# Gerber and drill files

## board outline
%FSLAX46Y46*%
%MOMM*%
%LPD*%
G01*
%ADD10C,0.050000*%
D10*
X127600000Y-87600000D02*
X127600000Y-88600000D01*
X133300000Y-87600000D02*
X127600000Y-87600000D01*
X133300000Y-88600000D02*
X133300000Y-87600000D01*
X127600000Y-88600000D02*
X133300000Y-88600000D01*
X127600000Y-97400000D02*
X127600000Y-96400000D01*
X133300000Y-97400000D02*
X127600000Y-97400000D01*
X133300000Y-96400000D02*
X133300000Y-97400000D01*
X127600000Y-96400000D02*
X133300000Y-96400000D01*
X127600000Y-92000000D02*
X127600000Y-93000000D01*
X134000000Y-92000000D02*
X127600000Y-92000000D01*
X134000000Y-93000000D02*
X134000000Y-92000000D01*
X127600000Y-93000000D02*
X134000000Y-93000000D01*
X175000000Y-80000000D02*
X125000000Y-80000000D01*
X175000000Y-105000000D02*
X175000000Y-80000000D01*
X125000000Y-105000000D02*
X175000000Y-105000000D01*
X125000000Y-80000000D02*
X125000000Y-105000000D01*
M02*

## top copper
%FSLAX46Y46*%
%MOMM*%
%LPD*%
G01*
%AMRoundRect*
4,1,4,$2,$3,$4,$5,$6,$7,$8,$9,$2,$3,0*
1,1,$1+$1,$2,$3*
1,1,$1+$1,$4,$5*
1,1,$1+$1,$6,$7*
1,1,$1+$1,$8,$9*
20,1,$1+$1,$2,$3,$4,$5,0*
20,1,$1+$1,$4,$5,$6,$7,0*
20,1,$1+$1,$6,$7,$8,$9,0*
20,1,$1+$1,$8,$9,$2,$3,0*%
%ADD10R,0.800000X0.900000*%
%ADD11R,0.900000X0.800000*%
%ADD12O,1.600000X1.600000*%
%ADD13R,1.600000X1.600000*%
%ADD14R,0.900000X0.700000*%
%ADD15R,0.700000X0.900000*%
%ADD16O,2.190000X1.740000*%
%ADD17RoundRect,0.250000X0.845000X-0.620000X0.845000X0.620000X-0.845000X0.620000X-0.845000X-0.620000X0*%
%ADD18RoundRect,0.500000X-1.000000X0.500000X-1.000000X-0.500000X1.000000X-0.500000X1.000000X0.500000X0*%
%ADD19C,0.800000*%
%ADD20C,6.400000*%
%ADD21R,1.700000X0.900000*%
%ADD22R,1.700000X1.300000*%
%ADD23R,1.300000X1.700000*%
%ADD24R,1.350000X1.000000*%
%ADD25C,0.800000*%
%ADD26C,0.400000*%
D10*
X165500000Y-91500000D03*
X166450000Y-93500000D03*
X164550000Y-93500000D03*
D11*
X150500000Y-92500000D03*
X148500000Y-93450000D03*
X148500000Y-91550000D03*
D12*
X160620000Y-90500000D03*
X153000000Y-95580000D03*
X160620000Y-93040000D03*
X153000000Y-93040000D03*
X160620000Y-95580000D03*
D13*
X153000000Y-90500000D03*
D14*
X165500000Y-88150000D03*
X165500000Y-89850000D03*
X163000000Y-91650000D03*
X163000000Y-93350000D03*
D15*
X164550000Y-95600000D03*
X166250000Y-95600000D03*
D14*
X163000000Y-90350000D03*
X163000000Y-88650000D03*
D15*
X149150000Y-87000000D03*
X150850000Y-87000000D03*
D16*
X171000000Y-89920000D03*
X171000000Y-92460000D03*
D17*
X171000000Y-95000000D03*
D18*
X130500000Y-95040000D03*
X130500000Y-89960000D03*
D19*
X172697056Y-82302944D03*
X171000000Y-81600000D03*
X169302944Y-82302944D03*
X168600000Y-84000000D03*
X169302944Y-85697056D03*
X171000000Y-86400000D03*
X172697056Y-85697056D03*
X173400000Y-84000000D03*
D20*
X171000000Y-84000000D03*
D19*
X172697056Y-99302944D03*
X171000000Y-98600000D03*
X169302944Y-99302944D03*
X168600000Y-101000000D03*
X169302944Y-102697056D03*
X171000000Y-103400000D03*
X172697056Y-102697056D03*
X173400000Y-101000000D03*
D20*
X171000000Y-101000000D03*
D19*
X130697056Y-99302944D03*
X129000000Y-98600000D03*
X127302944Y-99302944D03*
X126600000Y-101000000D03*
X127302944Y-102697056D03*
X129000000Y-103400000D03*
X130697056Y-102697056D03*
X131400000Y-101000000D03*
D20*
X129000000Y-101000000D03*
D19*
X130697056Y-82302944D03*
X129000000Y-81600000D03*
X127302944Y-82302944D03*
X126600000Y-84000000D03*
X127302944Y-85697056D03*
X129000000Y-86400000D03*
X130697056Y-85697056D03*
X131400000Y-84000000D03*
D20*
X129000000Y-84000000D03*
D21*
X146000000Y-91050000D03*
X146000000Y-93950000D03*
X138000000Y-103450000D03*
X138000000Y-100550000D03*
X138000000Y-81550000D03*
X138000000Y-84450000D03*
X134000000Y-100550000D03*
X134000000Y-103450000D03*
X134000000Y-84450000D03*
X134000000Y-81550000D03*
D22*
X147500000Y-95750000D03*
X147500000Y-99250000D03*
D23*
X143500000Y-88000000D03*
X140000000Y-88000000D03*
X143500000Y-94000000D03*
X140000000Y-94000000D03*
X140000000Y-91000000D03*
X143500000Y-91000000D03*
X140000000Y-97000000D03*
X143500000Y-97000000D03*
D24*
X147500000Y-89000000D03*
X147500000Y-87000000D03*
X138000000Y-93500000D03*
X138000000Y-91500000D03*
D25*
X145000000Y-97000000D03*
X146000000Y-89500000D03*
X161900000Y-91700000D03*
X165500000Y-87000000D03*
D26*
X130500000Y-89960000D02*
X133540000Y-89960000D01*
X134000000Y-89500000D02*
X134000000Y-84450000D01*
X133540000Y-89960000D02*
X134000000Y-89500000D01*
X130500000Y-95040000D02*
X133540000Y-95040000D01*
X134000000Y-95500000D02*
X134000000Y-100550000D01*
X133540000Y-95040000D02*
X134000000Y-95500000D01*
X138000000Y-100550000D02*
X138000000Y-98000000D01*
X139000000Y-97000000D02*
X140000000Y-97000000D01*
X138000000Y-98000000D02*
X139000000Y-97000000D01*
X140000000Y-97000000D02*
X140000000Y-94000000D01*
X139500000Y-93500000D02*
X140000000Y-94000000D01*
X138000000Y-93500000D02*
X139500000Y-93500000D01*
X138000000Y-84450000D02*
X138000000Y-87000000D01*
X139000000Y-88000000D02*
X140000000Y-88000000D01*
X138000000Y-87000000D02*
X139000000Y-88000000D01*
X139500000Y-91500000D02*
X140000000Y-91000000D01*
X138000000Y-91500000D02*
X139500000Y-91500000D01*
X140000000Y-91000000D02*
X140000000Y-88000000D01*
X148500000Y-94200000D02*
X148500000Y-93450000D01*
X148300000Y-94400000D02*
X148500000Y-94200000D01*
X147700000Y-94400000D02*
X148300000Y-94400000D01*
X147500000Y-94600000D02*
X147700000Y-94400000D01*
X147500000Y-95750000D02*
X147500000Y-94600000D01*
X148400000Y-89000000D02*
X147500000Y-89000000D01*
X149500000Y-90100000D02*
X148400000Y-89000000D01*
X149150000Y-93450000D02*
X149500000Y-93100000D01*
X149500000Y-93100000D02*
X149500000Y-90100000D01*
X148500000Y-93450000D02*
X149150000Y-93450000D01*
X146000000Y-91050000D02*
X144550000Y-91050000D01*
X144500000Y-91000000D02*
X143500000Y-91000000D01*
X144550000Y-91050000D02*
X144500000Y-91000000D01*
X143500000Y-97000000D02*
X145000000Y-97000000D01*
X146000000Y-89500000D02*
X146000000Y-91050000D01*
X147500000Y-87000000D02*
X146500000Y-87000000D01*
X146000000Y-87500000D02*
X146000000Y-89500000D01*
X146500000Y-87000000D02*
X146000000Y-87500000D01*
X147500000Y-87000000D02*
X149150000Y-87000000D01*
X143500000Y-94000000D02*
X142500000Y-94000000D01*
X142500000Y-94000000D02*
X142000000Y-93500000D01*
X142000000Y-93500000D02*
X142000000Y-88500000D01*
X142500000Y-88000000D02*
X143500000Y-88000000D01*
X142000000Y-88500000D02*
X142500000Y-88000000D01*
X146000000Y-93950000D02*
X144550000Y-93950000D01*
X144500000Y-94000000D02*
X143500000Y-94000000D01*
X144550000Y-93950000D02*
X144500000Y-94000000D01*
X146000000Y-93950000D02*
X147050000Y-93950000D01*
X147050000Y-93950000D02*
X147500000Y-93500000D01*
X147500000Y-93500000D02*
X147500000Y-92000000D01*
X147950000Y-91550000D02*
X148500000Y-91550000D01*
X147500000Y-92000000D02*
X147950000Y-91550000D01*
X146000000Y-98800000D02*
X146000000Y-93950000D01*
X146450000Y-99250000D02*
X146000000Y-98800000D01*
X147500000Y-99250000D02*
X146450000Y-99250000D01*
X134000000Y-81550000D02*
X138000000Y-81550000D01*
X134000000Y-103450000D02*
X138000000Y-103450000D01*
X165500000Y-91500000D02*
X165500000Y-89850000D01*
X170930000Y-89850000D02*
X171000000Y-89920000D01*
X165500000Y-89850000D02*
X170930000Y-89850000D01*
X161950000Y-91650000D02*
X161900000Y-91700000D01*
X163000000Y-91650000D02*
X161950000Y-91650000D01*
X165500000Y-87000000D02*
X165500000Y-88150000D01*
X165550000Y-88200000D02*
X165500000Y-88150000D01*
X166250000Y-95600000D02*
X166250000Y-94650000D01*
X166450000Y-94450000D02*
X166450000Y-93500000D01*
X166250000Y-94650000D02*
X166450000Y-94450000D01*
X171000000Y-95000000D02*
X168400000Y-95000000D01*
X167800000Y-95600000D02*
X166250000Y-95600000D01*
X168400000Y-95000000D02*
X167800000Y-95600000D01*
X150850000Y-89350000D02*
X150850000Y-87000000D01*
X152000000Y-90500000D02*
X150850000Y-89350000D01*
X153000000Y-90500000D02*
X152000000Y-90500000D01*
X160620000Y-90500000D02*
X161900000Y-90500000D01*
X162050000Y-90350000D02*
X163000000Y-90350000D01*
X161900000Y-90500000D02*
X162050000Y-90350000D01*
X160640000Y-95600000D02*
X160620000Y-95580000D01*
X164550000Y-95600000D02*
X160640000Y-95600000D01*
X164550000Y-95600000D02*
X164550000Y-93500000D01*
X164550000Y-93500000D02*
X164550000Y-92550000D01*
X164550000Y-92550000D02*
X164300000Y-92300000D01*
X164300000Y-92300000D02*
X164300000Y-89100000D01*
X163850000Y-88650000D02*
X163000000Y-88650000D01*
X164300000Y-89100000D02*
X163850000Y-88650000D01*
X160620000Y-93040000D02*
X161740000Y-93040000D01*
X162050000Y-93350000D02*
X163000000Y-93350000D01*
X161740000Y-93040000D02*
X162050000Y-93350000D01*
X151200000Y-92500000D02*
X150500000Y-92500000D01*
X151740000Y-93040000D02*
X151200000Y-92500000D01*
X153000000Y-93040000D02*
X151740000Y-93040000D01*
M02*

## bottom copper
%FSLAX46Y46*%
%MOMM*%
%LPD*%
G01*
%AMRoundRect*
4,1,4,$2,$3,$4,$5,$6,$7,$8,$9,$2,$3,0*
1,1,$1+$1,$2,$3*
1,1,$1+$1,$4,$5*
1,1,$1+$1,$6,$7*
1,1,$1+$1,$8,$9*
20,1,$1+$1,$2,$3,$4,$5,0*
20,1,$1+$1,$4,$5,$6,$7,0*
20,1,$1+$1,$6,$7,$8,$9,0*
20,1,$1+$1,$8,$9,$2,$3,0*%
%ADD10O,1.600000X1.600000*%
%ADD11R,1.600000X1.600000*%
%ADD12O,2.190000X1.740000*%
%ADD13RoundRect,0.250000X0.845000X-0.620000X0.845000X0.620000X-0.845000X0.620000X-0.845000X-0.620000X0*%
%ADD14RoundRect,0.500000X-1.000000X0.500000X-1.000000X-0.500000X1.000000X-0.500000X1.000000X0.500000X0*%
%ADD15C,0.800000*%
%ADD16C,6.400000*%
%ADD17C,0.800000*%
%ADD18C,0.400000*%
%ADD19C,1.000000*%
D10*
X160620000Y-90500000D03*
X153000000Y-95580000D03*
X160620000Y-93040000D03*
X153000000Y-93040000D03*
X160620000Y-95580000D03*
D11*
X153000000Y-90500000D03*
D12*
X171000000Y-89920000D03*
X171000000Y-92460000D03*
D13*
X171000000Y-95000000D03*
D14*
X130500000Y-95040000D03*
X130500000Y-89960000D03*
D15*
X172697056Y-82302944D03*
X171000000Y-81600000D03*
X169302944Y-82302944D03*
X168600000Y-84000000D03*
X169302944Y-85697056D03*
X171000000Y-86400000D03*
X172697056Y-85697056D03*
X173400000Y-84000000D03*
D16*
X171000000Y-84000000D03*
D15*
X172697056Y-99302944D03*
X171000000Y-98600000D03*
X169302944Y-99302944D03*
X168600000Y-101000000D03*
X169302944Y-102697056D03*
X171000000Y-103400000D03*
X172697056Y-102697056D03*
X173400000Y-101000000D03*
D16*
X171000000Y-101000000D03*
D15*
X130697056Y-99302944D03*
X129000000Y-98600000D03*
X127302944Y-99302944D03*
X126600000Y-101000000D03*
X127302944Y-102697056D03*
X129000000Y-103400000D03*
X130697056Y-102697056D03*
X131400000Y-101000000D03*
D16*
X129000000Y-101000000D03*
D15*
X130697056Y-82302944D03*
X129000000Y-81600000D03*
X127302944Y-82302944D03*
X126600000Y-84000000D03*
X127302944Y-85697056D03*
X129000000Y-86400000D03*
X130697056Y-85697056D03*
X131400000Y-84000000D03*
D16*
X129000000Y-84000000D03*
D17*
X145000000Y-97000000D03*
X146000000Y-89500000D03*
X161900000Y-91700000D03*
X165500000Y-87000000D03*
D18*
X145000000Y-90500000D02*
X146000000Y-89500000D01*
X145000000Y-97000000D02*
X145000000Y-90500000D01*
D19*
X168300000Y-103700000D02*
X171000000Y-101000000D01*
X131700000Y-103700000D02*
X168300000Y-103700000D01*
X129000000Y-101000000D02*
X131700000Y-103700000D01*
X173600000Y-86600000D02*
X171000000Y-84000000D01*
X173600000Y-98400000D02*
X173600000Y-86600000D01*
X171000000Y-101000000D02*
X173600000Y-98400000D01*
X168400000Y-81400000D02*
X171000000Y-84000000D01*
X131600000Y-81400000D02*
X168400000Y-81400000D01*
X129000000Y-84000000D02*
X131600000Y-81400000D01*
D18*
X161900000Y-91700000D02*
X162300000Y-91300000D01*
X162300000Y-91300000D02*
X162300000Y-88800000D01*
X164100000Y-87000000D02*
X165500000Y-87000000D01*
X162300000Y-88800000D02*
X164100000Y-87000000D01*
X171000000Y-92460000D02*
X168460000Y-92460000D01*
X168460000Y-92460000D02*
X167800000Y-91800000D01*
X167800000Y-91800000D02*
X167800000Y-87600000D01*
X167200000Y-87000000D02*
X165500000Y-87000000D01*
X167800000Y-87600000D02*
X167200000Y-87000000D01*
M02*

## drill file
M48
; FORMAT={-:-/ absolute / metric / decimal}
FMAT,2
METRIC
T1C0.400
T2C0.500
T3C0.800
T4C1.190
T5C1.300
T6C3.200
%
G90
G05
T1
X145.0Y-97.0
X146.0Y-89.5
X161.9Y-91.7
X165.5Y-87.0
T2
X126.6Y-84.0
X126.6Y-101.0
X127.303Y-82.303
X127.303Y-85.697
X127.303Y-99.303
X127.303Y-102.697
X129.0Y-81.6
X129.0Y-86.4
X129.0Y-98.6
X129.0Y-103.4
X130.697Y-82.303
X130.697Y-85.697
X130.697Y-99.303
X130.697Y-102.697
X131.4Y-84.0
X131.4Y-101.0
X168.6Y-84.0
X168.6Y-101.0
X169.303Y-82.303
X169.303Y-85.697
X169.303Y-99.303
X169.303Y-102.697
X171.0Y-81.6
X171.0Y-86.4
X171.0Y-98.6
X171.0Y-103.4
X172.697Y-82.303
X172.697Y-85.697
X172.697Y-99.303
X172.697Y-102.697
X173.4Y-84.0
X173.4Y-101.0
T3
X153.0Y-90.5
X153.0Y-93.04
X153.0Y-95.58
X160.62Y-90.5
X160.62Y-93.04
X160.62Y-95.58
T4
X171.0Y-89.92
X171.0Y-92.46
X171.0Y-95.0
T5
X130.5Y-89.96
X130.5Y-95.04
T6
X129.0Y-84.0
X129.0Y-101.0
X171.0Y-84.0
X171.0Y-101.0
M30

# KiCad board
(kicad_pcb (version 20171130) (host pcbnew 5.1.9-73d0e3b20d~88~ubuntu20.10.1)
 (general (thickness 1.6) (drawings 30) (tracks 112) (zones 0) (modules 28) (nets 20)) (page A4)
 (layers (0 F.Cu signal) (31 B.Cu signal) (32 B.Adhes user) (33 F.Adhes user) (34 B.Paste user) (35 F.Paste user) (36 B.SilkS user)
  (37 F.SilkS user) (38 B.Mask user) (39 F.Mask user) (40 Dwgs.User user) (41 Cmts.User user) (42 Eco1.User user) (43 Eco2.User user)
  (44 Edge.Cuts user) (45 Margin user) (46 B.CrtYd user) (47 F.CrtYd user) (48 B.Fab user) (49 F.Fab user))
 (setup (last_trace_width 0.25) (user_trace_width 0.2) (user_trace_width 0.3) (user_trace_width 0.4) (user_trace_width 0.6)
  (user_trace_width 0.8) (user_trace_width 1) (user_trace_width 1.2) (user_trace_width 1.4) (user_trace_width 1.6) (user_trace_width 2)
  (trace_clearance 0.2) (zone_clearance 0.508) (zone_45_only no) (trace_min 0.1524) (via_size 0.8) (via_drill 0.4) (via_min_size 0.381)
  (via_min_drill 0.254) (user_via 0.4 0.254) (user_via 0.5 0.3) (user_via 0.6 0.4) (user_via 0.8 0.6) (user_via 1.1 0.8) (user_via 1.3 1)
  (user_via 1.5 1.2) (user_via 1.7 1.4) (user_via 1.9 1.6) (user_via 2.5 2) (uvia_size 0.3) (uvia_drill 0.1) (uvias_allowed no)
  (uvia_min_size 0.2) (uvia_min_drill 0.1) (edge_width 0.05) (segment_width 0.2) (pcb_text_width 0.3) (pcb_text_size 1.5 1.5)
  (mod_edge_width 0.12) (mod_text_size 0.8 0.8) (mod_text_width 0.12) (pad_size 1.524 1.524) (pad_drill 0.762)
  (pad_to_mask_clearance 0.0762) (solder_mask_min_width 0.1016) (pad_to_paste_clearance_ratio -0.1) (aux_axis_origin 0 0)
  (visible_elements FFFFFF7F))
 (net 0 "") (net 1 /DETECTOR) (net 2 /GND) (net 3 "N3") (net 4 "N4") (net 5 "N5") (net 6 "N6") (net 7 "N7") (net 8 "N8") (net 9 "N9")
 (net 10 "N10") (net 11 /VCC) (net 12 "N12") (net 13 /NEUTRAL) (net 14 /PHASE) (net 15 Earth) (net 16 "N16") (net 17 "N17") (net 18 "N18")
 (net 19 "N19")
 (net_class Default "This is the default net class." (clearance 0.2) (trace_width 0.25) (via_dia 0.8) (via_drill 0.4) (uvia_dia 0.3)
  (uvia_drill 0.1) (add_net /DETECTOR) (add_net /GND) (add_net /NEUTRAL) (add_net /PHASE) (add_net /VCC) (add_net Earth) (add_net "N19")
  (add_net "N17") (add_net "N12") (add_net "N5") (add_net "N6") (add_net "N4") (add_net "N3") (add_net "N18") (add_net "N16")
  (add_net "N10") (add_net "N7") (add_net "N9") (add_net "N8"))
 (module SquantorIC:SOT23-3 (layer F.Cu) (at 165.5 92.5)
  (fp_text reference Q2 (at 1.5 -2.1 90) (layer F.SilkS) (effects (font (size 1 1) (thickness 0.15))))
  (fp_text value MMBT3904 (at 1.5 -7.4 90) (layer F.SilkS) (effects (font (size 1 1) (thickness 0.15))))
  (pad 3 smd rect (at 0 -1) (size 0.8 0.9) (layers F.Cu F.Paste F.Mask) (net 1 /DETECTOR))
  (pad 2 smd rect (at 0.95 1) (size 0.8 0.9) (layers F.Cu F.Paste F.Mask) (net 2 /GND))
  (pad 1 smd rect (at -0.95 1) (size 0.8 0.9) (layers F.Cu F.Paste F.Mask) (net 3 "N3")))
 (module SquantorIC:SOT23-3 (layer F.Cu) (at 149.5 92.5 270)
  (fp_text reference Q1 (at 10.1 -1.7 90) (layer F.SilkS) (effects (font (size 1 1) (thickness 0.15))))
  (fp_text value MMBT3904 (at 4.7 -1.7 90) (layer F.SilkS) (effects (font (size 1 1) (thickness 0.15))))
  (pad 3 smd rect (at 0 -1 270) (size 0.8 0.9) (layers F.Cu F.Paste F.Mask) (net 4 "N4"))
  (pad 2 smd rect (at 0.95 1 270) (size 0.8 0.9) (layers F.Cu F.Paste F.Mask) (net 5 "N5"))
  (pad 1 smd rect (at -0.95 1 270) (size 0.8 0.9) (layers F.Cu F.Paste F.Mask) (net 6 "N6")))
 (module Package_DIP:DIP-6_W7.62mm (layer F.Cu) (at 153 90.5)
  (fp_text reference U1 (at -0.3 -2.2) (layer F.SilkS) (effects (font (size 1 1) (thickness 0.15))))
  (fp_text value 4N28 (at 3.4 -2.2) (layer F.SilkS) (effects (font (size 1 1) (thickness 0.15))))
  (pad 6 thru_hole oval (at 7.62 0) (size 1.6 1.6) (drill 0.8) (layers *.Cu *.Mask) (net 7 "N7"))
  (pad 3 thru_hole oval (at 0 5.08) (size 1.6 1.6) (drill 0.8) (layers *.Cu *.Mask) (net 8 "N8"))
  (pad 5 thru_hole oval (at 7.62 2.54) (size 1.6 1.6) (drill 0.8) (layers *.Cu *.Mask) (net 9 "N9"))
  (pad 2 thru_hole oval (at 0 2.54) (size 1.6 1.6) (drill 0.8) (layers *.Cu *.Mask) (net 4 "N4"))
  (pad 4 thru_hole oval (at 7.62 5.08) (size 1.6 1.6) (drill 0.8) (layers *.Cu *.Mask) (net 3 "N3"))
  (pad 1 thru_hole rect (at 0 0) (size 1.6 1.6) (drill 0.8) (layers *.Cu *.Mask) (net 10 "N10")))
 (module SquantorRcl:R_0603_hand (layer F.Cu) (at 165.5 89 90)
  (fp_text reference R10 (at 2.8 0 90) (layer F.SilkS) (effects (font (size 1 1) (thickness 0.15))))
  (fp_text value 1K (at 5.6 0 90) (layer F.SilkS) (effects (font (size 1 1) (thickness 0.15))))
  (pad 2 smd rect (at 0.85 0 90) (size 0.7 0.9) (layers F.Cu F.Paste F.Mask) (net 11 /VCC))
  (pad 1 smd rect (at -0.85 0 90) (size 0.7 0.9) (layers F.Cu F.Paste F.Mask) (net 1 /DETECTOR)))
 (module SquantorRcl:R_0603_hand (layer F.Cu) (at 163 92.5 90)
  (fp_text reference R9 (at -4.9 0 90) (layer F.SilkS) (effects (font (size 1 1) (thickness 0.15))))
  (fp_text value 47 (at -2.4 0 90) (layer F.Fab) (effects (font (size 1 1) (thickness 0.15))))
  (pad 2 smd rect (at 0.85 0 90) (size 0.7 0.9) (layers F.Cu F.Paste F.Mask) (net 11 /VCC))
  (pad 1 smd rect (at -0.85 0 90) (size 0.7 0.9) (layers F.Cu F.Paste F.Mask) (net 9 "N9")))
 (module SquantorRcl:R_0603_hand (layer F.Cu) (at 165.4 95.6 180)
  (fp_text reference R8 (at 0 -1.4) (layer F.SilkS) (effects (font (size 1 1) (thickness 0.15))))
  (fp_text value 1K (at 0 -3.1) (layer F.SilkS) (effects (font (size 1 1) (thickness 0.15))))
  (pad 2 smd rect (at 0.85 0 180) (size 0.7 0.9) (layers F.Cu F.Paste F.Mask) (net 3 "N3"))
  (pad 1 smd rect (at -0.85 0 180) (size 0.7 0.9) (layers F.Cu F.Paste F.Mask) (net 2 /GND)))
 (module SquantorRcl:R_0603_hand (layer F.Cu) (at 163 89.5 270)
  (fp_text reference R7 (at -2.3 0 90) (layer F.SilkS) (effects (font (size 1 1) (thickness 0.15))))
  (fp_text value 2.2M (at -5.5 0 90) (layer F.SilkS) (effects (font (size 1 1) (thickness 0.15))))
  (pad 2 smd rect (at 0.85 0 270) (size 0.7 0.9) (layers F.Cu F.Paste F.Mask) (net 7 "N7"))
  (pad 1 smd rect (at -0.85 0 270) (size 0.7 0.9) (layers F.Cu F.Paste F.Mask) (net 3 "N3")))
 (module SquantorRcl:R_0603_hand (layer F.Cu) (at 150 87 180)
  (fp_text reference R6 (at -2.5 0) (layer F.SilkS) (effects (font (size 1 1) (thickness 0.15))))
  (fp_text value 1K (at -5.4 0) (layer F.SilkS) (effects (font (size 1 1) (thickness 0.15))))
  (pad 2 smd rect (at 0.85 0 180) (size 0.7 0.9) (layers F.Cu F.Paste F.Mask) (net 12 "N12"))
  (pad 1 smd rect (at -0.85 0 180) (size 0.7 0.9) (layers F.Cu F.Paste F.Mask) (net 10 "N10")))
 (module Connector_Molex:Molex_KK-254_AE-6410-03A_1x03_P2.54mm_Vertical (layer F.Cu) (at 171 95 90)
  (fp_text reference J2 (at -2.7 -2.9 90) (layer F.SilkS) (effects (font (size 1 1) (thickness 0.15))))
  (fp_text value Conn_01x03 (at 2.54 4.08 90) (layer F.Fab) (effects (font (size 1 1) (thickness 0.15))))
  (pad 3 thru_hole oval (at 5.08 0 90) (size 1.74 2.19) (drill 1.19) (layers *.Cu *.Mask) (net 1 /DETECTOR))
  (pad 2 thru_hole oval (at 2.54 0 90) (size 1.74 2.19) (drill 1.19) (layers *.Cu *.Mask) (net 11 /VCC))
  (pad 1 thru_hole roundrect (at 0 0 90) (size 1.74 2.19) (drill 1.19) (layers *.Cu *.Mask) (roundrect_rratio 0.143678) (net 2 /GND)))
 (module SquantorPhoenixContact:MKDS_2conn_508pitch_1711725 (layer F.Cu) (at 130.5 92.5 270)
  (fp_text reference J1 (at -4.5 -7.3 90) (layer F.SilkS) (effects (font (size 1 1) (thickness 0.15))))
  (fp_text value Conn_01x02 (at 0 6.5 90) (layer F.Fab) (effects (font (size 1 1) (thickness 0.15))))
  (pad 2 thru_hole roundrect (at 2.54 0 270) (size 2 3) (drill 1.3) (layers *.Cu *.Mask) (roundrect_rratio 0.25) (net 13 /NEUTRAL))
  (pad 1 thru_hole roundrect (at -2.54 0 270) (size 2 3) (drill 1.3) (layers *.Cu *.Mask) (roundrect_rratio 0.25) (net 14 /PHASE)))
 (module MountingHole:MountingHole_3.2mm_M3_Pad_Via (layer F.Cu) (at 171 84)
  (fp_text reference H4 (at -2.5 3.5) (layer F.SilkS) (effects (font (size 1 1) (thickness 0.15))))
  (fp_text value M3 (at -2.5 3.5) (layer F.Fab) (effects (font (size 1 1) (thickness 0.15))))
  (pad 1 thru_hole circle (at 1.697056 -1.697056) (size 0.8 0.8) (drill 0.5) (layers *.Cu *.Mask) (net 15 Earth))
  (pad 1 thru_hole circle (at 0 -2.4) (size 0.8 0.8) (drill 0.5) (layers *.Cu *.Mask) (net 15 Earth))
  (pad 1 thru_hole circle (at -1.697056 -1.697056) (size 0.8 0.8) (drill 0.5) (layers *.Cu *.Mask) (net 15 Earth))
  (pad 1 thru_hole circle (at -2.4 0) (size 0.8 0.8) (drill 0.5) (layers *.Cu *.Mask) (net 15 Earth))
  (pad 1 thru_hole circle (at -1.697056 1.697056) (size 0.8 0.8) (drill 0.5) (layers *.Cu *.Mask) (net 15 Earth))
  (pad 1 thru_hole circle (at 0 2.4) (size 0.8 0.8) (drill 0.5) (layers *.Cu *.Mask) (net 15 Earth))
  (pad 1 thru_hole circle (at 1.697056 1.697056) (size 0.8 0.8) (drill 0.5) (layers *.Cu *.Mask) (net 15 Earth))
  (pad 1 thru_hole circle (at 2.4 0) (size 0.8 0.8) (drill 0.5) (layers *.Cu *.Mask) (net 15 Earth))
  (pad 1 thru_hole circle (at 0 0) (size 6.4 6.4) (drill 3.2) (layers *.Cu *.Mask) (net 15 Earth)))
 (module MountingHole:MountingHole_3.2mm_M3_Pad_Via (layer F.Cu) (at 171 101)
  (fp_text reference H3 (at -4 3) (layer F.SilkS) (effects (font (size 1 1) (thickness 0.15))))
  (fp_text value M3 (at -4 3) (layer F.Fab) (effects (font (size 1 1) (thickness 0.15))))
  (pad 1 thru_hole circle (at 1.697056 -1.697056) (size 0.8 0.8) (drill 0.5) (layers *.Cu *.Mask) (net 15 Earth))
  (pad 1 thru_hole circle (at 0 -2.4) (size 0.8 0.8) (drill 0.5) (layers *.Cu *.Mask) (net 15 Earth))
  (pad 1 thru_hole circle (at -1.697056 -1.697056) (size 0.8 0.8) (drill 0.5) (layers *.Cu *.Mask) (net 15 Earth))
  (pad 1 thru_hole circle (at -2.4 0) (size 0.8 0.8) (drill 0.5) (layers *.Cu *.Mask) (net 15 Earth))
  (pad 1 thru_hole circle (at -1.697056 1.697056) (size 0.8 0.8) (drill 0.5) (layers *.Cu *.Mask) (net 15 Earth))
  (pad 1 thru_hole circle (at 0 2.4) (size 0.8 0.8) (drill 0.5) (layers *.Cu *.Mask) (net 15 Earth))
  (pad 1 thru_hole circle (at 1.697056 1.697056) (size 0.8 0.8) (drill 0.5) (layers *.Cu *.Mask) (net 15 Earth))
  (pad 1 thru_hole circle (at 2.4 0) (size 0.8 0.8) (drill 0.5) (layers *.Cu *.Mask) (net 15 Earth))
  (pad 1 thru_hole circle (at 0 0) (size 6.4 6.4) (drill 3.2) (layers *.Cu *.Mask) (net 15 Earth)))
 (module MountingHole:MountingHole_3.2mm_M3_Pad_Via (layer F.Cu) (at 129 101)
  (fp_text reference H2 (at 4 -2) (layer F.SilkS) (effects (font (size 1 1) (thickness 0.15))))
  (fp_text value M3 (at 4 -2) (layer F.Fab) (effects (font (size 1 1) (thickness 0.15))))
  (pad 1 thru_hole circle (at 1.697056 -1.697056) (size 0.8 0.8) (drill 0.5) (layers *.Cu *.Mask) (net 15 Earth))
  (pad 1 thru_hole circle (at 0 -2.4) (size 0.8 0.8) (drill 0.5) (layers *.Cu *.Mask) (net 15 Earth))
  (pad 1 thru_hole circle (at -1.697056 -1.697056) (size 0.8 0.8) (drill 0.5) (layers *.Cu *.Mask) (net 15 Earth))
  (pad 1 thru_hole circle (at -2.4 0) (size 0.8 0.8) (drill 0.5) (layers *.Cu *.Mask) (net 15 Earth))
  (pad 1 thru_hole circle (at -1.697056 1.697056) (size 0.8 0.8) (drill 0.5) (layers *.Cu *.Mask) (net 15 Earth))
  (pad 1 thru_hole circle (at 0 2.4) (size 0.8 0.8) (drill 0.5) (layers *.Cu *.Mask) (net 15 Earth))
  (pad 1 thru_hole circle (at 1.697056 1.697056) (size 0.8 0.8) (drill 0.5) (layers *.Cu *.Mask) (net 15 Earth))
  (pad 1 thru_hole circle (at 2.4 0) (size 0.8 0.8) (drill 0.5) (layers *.Cu *.Mask) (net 15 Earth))
  (pad 1 thru_hole circle (at 0 0) (size 6.4 6.4) (drill 3.2) (layers *.Cu *.Mask) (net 15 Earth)))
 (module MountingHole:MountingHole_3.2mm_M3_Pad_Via (layer F.Cu) (at 129 84)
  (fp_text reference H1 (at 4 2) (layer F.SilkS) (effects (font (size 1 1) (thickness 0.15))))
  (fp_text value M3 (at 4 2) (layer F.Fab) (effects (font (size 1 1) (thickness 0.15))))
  (pad 1 thru_hole circle (at 1.697056 -1.697056) (size 0.8 0.8) (drill 0.5) (layers *.Cu *.Mask) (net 15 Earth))
  (pad 1 thru_hole circle (at 0 -2.4) (size 0.8 0.8) (drill 0.5) (layers *.Cu *.Mask) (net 15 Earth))
  (pad 1 thru_hole circle (at -1.697056 -1.697056) (size 0.8 0.8) (drill 0.5) (layers *.Cu *.Mask) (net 15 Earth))
  (pad 1 thru_hole circle (at -2.4 0) (size 0.8 0.8) (drill 0.5) (layers *.Cu *.Mask) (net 15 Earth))
  (pad 1 thru_hole circle (at -1.697056 1.697056) (size 0.8 0.8) (drill 0.5) (layers *.Cu *.Mask) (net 15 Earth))
  (pad 1 thru_hole circle (at 0 2.4) (size 0.8 0.8) (drill 0.5) (layers *.Cu *.Mask) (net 15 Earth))
  (pad 1 thru_hole circle (at 1.697056 1.697056) (size 0.8 0.8) (drill 0.5) (layers *.Cu *.Mask) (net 15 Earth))
  (pad 1 thru_hole circle (at 2.4 0) (size 0.8 0.8) (drill 0.5) (layers *.Cu *.Mask) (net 15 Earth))
  (pad 1 thru_hole circle (at 0 0) (size 6.4 6.4) (drill 3.2) (layers *.Cu *.Mask) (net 15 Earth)))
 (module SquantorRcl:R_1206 (layer F.Cu) (at 146 92.5 90)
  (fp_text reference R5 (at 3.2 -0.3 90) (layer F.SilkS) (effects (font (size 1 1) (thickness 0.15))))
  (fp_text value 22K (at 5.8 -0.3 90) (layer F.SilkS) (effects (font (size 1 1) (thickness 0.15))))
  (pad 2 smd rect (at 1.45 0 90) (size 0.9 1.7) (layers F.Cu F.Paste F.Mask) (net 12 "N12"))
  (pad 1 smd rect (at -1.45 0 90) (size 0.9 1.7) (layers F.Cu F.Paste F.Mask) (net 6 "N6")))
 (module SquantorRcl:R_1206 (layer F.Cu) (at 138 102 270)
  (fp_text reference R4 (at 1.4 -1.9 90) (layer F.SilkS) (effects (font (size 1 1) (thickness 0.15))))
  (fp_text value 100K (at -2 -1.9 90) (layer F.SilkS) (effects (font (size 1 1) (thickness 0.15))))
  (pad 2 smd rect (at 1.45 0 270) (size 0.9 1.7) (layers F.Cu F.Paste F.Mask) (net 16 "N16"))
  (pad 1 smd rect (at -1.45 0 270) (size 0.9 1.7) (layers F.Cu F.Paste F.Mask) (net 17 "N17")))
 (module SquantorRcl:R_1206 (layer F.Cu) (at 138 83 90)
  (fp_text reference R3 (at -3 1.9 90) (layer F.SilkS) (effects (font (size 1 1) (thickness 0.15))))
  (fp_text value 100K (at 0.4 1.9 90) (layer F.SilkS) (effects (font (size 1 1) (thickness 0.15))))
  (pad 2 smd rect (at 1.45 0 90) (size 0.9 1.7) (layers F.Cu F.Paste F.Mask) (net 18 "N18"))
  (pad 1 smd rect (at -1.45 0 90) (size 0.9 1.7) (layers F.Cu F.Paste F.Mask) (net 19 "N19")))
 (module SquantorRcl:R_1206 (layer F.Cu) (at 134 102 90)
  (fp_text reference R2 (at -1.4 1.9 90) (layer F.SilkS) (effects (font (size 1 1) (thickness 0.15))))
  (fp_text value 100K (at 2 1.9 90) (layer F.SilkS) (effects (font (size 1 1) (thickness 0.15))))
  (pad 2 smd rect (at 1.45 0 90) (size 0.9 1.7) (layers F.Cu F.Paste F.Mask) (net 13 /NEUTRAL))
  (pad 1 smd rect (at -1.45 0 90) (size 0.9 1.7) (layers F.Cu F.Paste F.Mask) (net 16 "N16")))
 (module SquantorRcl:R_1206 (layer F.Cu) (at 134 83 270)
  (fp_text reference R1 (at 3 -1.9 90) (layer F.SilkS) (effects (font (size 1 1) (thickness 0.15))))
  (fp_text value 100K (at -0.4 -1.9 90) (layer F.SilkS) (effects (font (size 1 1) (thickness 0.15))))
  (pad 2 smd rect (at 1.45 0 270) (size 0.9 1.7) (layers F.Cu F.Paste F.Mask) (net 14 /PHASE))
  (pad 1 smd rect (at -1.45 0 270) (size 0.9 1.7) (layers F.Cu F.Paste F.Mask) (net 18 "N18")))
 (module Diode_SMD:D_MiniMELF (layer F.Cu) (at 147.5 97.5 90)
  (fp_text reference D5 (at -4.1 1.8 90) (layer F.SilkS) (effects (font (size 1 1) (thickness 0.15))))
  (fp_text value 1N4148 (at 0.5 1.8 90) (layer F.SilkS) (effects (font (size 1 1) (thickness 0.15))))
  (pad 2 smd rect (at 1.75 0 90) (size 1.3 1.7) (layers F.Cu F.Paste F.Mask) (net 5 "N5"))
  (pad 1 smd rect (at -1.75 0 90) (size 1.3 1.7) (layers F.Cu F.Paste F.Mask) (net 6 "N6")))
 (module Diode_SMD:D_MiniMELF (layer F.Cu) (at 141.75 88)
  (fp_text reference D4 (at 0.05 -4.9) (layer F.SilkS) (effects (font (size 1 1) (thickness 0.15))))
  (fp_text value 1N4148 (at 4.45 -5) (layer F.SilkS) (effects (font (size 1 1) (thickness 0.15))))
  (pad 2 smd rect (at 1.75 0) (size 1.3 1.7) (layers F.Cu F.Paste F.Mask) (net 6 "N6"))
  (pad 1 smd rect (at -1.75 0) (size 1.3 1.7) (layers F.Cu F.Paste F.Mask) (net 19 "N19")))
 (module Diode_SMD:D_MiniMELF (layer F.Cu) (at 141.75 94)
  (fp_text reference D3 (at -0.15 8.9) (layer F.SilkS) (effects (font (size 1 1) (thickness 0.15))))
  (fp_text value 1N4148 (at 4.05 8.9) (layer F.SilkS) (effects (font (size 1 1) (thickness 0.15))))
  (pad 2 smd rect (at 1.75 0) (size 1.3 1.7) (layers F.Cu F.Paste F.Mask) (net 6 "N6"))
  (pad 1 smd rect (at -1.75 0) (size 1.3 1.7) (layers F.Cu F.Paste F.Mask) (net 17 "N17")))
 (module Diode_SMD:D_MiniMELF (layer F.Cu) (at 141.75 91 180)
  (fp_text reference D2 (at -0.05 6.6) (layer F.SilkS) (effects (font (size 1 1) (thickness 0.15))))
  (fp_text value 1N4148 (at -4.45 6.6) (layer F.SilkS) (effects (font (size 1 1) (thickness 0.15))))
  (pad 2 smd rect (at 1.75 0 180) (size 1.3 1.7) (layers F.Cu F.Paste F.Mask) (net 19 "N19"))
  (pad 1 smd rect (at -1.75 0 180) (size 1.3 1.7) (layers F.Cu F.Paste F.Mask) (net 12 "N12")))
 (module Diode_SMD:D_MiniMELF (layer F.Cu) (at 141.75 97 180)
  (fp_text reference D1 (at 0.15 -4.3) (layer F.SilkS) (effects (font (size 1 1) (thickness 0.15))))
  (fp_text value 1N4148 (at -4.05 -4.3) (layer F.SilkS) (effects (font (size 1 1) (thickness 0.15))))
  (pad 2 smd rect (at 1.75 0 180) (size 1.3 1.7) (layers F.Cu F.Paste F.Mask) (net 17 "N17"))
  (pad 1 smd rect (at -1.75 0 180) (size 1.3 1.7) (layers F.Cu F.Paste F.Mask) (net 12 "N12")))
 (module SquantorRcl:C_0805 (layer F.Cu) (at 147.5 88 270)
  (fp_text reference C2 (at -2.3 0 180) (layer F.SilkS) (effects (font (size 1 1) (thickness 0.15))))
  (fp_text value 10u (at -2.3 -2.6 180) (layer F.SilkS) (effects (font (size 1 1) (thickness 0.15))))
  (pad 2 smd rect (at 1 0 270) (size 1 1.35) (layers F.Cu F.Paste F.Mask) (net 5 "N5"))
  (pad 1 smd rect (at -1 0 270) (size 1 1.35) (layers F.Cu F.Paste F.Mask) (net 12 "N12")))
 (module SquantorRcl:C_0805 (layer F.Cu) (at 138 92.5 270)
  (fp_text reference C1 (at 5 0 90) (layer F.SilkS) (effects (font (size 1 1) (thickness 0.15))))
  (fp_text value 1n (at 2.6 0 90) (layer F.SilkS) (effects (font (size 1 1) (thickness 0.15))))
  (pad 2 smd rect (at 1 0 270) (size 1 1.35) (layers F.Cu F.Paste F.Mask) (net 17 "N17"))
  (pad 1 smd rect (at -1 0 270) (size 1 1.35) (layers F.Cu F.Paste F.Mask) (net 19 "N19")))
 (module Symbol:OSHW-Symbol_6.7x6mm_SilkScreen (layer B.Cu) (at 156.9 98.7 180)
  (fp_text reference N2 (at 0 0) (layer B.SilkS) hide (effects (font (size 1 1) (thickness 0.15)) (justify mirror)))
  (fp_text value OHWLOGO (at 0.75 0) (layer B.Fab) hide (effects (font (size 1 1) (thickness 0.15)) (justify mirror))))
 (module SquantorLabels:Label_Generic (layer B.Cu) (at 157.5 102.6 180)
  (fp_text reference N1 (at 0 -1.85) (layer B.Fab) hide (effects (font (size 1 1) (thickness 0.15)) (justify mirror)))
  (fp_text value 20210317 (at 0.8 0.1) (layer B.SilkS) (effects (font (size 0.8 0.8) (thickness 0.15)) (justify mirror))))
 (gr_line (start 127.6 87.6) (end 127.6 88.6) (layer Edge.Cuts) (width 0.05))
 (gr_line (start 133.3 87.6) (end 127.6 87.6) (layer Edge.Cuts) (width 0.05))
 (gr_line (start 133.3 88.6) (end 133.3 87.6) (layer Edge.Cuts) (width 0.05))
 (gr_line (start 127.6 88.6) (end 133.3 88.6) (layer Edge.Cuts) (width 0.05))
 (gr_line (start 127.6 97.4) (end 127.6 96.4) (layer Edge.Cuts) (width 0.05))
 (gr_line (start 133.3 97.4) (end 127.6 97.4) (layer Edge.Cuts) (width 0.05))
 (gr_line (start 133.3 96.4) (end 133.3 97.4) (layer Edge.Cuts) (width 0.05))
 (gr_line (start 127.6 96.4) (end 133.3 96.4) (layer Edge.Cuts) (width 0.05))
 (gr_line (start 127.6 92) (end 127.6 93) (layer Edge.Cuts) (width 0.05))
 (gr_line (start 134 92) (end 127.6 92) (layer Edge.Cuts) (width 0.05))
 (gr_line (start 134 93) (end 134 92) (layer Edge.Cuts) (width 0.05))
 (gr_line (start 127.6 93) (end 134 93) (layer Edge.Cuts) (width 0.05))
 (gr_line (start 175 80) (end 125 80) (layer Edge.Cuts) (width 0.05))
 (gr_line (start 175 105) (end 175 80) (layer Edge.Cuts) (width 0.05))
 (gr_line (start 125 105) (end 175 105) (layer Edge.Cuts) (width 0.05))
 (gr_line (start 125 80) (end 125 105) (layer Edge.Cuts) (width 0.05))
 (segment (start 130.5 89.96) (end 133.54 89.96) (width 0.4) (layer F.Cu) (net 14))
 (segment (start 134 89.5) (end 134 84.45) (width 0.4) (layer F.Cu) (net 14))
 (segment (start 133.54 89.96) (end 134 89.5) (width 0.4) (layer F.Cu) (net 14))
 (segment (start 130.5 95.04) (end 133.54 95.04) (width 0.4) (layer F.Cu) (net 13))
 (segment (start 134 95.5) (end 134 100.55) (width 0.4) (layer F.Cu) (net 13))
 (segment (start 133.54 95.04) (end 134 95.5) (width 0.4) (layer F.Cu) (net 13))
 (segment (start 138 100.55) (end 138 98) (width 0.4) (layer F.Cu) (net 17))
 (segment (start 139 97) (end 140 97) (width 0.4) (layer F.Cu) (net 17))
 (segment (start 138 98) (end 139 97) (width 0.4) (layer F.Cu) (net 17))
 (segment (start 140 97) (end 140 94) (width 0.4) (layer F.Cu) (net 17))
 (segment (start 139.5 93.5) (end 140 94) (width 0.4) (layer F.Cu) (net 17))
 (segment (start 138 93.5) (end 139.5 93.5) (width 0.4) (layer F.Cu) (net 17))
 (segment (start 138 84.45) (end 138 87) (width 0.4) (layer F.Cu) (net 19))
 (segment (start 139 88) (end 140 88) (width 0.4) (layer F.Cu) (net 19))
 (segment (start 138 87) (end 139 88) (width 0.4) (layer F.Cu) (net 19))
 (segment (start 139.5 91.5) (end 140 91) (width 0.4) (layer F.Cu) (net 19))
 (segment (start 138 91.5) (end 139.5 91.5) (width 0.4) (layer F.Cu) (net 19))
 (segment (start 140 91) (end 140 88) (width 0.4) (layer F.Cu) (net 19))
 (segment (start 148.5 94.2) (end 148.5 93.45) (width 0.4) (layer F.Cu) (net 5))
 (segment (start 148.3 94.4) (end 148.5 94.2) (width 0.4) (layer F.Cu) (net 5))
 (segment (start 147.7 94.4) (end 148.3 94.4) (width 0.4) (layer F.Cu) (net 5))
 (segment (start 147.5 94.6) (end 147.7 94.4) (width 0.4) (layer F.Cu) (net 5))
 (segment (start 147.5 95.75) (end 147.5 94.6) (width 0.4) (layer F.Cu) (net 5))
 (segment (start 148.4 89) (end 147.5 89) (width 0.4) (layer F.Cu) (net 5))
 (segment (start 149.5 90.1) (end 148.4 89) (width 0.4) (layer F.Cu) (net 5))
 (segment (start 149.15 93.45) (end 149.5 93.1) (width 0.4) (layer F.Cu) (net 5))
 (segment (start 149.5 93.1) (end 149.5 90.1) (width 0.4) (layer F.Cu) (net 5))
 (segment (start 148.5 93.45) (end 149.15 93.45) (width 0.4) (layer F.Cu) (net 5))
 (segment (start 146 91.05) (end 144.55 91.05) (width 0.4) (layer F.Cu) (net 12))
 (segment (start 144.5 91) (end 143.5 91) (width 0.4) (layer F.Cu) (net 12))
 (segment (start 144.55 91.05) (end 144.5 91) (width 0.4) (layer F.Cu) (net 12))
 (via (at 145 97) (size 0.8) (drill 0.4) (layers F.Cu B.Cu) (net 12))
 (segment (start 143.5 97) (end 145 97) (width 0.4) (layer F.Cu) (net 12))
 (via (at 146 89.5) (size 0.8) (drill 0.4) (layers F.Cu B.Cu) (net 12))
 (segment (start 145 90.5) (end 146 89.5) (width 0.4) (layer B.Cu) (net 12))
 (segment (start 145 97) (end 145 90.5) (width 0.4) (layer B.Cu) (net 12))
 (segment (start 146 89.5) (end 146 91.05) (width 0.4) (layer F.Cu) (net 12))
 (segment (start 147.5 87) (end 146.5 87) (width 0.4) (layer F.Cu) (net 12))
 (segment (start 146 87.5) (end 146 89.5) (width 0.4) (layer F.Cu) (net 12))
 (segment (start 146.5 87) (end 146 87.5) (width 0.4) (layer F.Cu) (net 12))
 (segment (start 147.5 87) (end 149.15 87) (width 0.4) (layer F.Cu) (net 12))
 (segment (start 143.5 94) (end 142.5 94) (width 0.4) (layer F.Cu) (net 6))
 (segment (start 142.5 94) (end 142 93.5) (width 0.4) (layer F.Cu) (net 6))
 (segment (start 142 93.5) (end 142 88.5) (width 0.4) (layer F.Cu) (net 6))
 (segment (start 142.5 88) (end 143.5 88) (width 0.4) (layer F.Cu) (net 6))
 (segment (start 142 88.5) (end 142.5 88) (width 0.4) (layer F.Cu) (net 6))
 (segment (start 146 93.95) (end 144.55 93.95) (width 0.4) (layer F.Cu) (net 6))
 (segment (start 144.5 94) (end 143.5 94) (width 0.4) (layer F.Cu) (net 6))
 (segment (start 144.55 93.95) (end 144.5 94) (width 0.4) (layer F.Cu) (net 6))
 (segment (start 146 93.95) (end 147.05 93.95) (width 0.4) (layer F.Cu) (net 6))
 (segment (start 147.05 93.95) (end 147.5 93.5) (width 0.4) (layer F.Cu) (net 6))
 (segment (start 147.5 93.5) (end 147.5 92) (width 0.4) (layer F.Cu) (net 6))
 (segment (start 147.95 91.55) (end 148.5 91.55) (width 0.4) (layer F.Cu) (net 6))
 (segment (start 147.5 92) (end 147.95 91.55) (width 0.4) (layer F.Cu) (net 6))
 (segment (start 146 98.8) (end 146 93.95) (width 0.4) (layer F.Cu) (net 6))
 (segment (start 146.45 99.25) (end 146 98.8) (width 0.4) (layer F.Cu) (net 6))
 (segment (start 147.5 99.25) (end 146.45 99.25) (width 0.4) (layer F.Cu) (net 6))
 (segment (start 134 81.55) (end 138 81.55) (width 0.4) (layer F.Cu) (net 18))
 (segment (start 134 103.45) (end 138 103.45) (width 0.4) (layer F.Cu) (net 16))
 (segment (start 168.3 103.7) (end 171 101) (width 1) (layer B.Cu) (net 15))
 (segment (start 131.7 103.7) (end 168.3 103.7) (width 1) (layer B.Cu) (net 15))
 (segment (start 129 101) (end 131.7 103.7) (width 1) (layer B.Cu) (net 15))
 (segment (start 173.6 86.6) (end 171 84) (width 1) (layer B.Cu) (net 15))
 (segment (start 173.6 98.4) (end 173.6 86.6) (width 1) (layer B.Cu) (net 15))
 (segment (start 171 101) (end 173.6 98.4) (width 1) (layer B.Cu) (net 15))
 (segment (start 168.4 81.4) (end 171 84) (width 1) (layer B.Cu) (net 15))
 (segment (start 131.6 81.4) (end 168.4 81.4) (width 1) (layer B.Cu) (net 15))
 (segment (start 129 84) (end 131.6 81.4) (width 1) (layer B.Cu) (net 15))
 (segment (start 165.5 91.5) (end 165.5 89.85) (width 0.4) (layer F.Cu) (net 1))
 (segment (start 170.93 89.85) (end 171 89.92) (width 0.4) (layer F.Cu) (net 1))
 (segment (start 165.5 89.85) (end 170.93 89.85) (width 0.4) (layer F.Cu) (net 1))
 (via (at 161.9 91.7) (size 0.8) (drill 0.4) (layers F.Cu B.Cu) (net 11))
 (segment (start 161.95 91.65) (end 161.9 91.7) (width 0.4) (layer F.Cu) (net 11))
 (segment (start 163 91.65) (end 161.95 91.65) (width 0.4) (layer F.Cu) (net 11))
 (segment (start 161.9 91.7) (end 162.3 91.3) (width 0.4) (layer B.Cu) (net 11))
 (segment (start 162.3 91.3) (end 162.3 88.8) (width 0.4) (layer B.Cu) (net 11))
 (via (at 165.5 87) (size 0.8) (drill 0.4) (layers F.Cu B.Cu) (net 11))
 (segment (start 164.1 87) (end 165.5 87) (width 0.4) (layer B.Cu) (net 11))
 (segment (start 162.3 88.8) (end 164.1 87) (width 0.4) (layer B.Cu) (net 11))
 (segment (start 165.5 87) (end 165.5 88.15) (width 0.4) (layer F.Cu) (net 11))
 (segment (start 165.55 88.2) (end 165.5 88.15) (width 0.4) (layer F.Cu) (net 11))
 (segment (start 171 92.46) (end 168.46 92.46) (width 0.4) (layer B.Cu) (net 11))
 (segment (start 168.46 92.46) (end 167.8 91.8) (width 0.4) (layer B.Cu) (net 11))
 (segment (start 167.8 91.8) (end 167.8 87.6) (width 0.4) (layer B.Cu) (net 11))
 (segment (start 167.2 87) (end 165.5 87) (width 0.4) (layer B.Cu) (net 11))
 (segment (start 167.8 87.6) (end 167.2 87) (width 0.4) (layer B.Cu) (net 11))
 (segment (start 166.25 95.6) (end 166.25 94.65) (width 0.4) (layer F.Cu) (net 2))
 (segment (start 166.45 94.45) (end 166.45 93.5) (width 0.4) (layer F.Cu) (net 2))
 (segment (start 166.25 94.65) (end 166.45 94.45) (width 0.4) (layer F.Cu) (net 2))
 (segment (start 171 95) (end 168.4 95) (width 0.4) (layer F.Cu) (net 2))
 (segment (start 167.8 95.6) (end 166.25 95.6) (width 0.4) (layer F.Cu) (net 2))
 (segment (start 168.4 95) (end 167.8 95.6) (width 0.4) (layer F.Cu) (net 2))
 (segment (start 150.85 89.35) (end 150.85 87) (width 0.4) (layer F.Cu) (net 10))
 (segment (start 152 90.5) (end 150.85 89.35) (width 0.4) (layer F.Cu) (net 10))
 (segment (start 153 90.5) (end 152 90.5) (width 0.4) (layer F.Cu) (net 10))
 (segment (start 160.62 90.5) (end 161.9 90.5) (width 0.4) (layer F.Cu) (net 7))
 (segment (start 162.05 90.35) (end 163 90.35) (width 0.4) (layer F.Cu) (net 7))
 (segment (start 161.9 90.5) (end 162.05 90.35) (width 0.4) (layer F.Cu) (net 7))
 (segment (start 160.64 95.6) (end 160.62 95.58) (width 0.4) (layer F.Cu) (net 3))
 (segment (start 164.55 95.6) (end 160.64 95.6) (width 0.4) (layer F.Cu) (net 3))
 (segment (start 164.55 95.6) (end 164.55 93.5) (width 0.4) (layer F.Cu) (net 3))
 (segment (start 164.55 93.5) (end 164.55 92.55) (width 0.4) (layer F.Cu) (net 3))
 (segment (start 164.55 92.55) (end 164.3 92.3) (width 0.4) (layer F.Cu) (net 3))
 (segment (start 164.3 92.3) (end 164.3 89.1) (width 0.4) (layer F.Cu) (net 3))
 (segment (start 163.85 88.65) (end 163 88.65) (width 0.4) (layer F.Cu) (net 3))
 (segment (start 164.3 89.1) (end 163.85 88.65) (width 0.4) (layer F.Cu) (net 3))
 (segment (start 160.62 93.04) (end 161.74 93.04) (width 0.4) (layer F.Cu) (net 9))
 (segment (start 162.05 93.35) (end 163 93.35) (width 0.4) (layer F.Cu) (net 9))
 (segment (start 161.74 93.04) (end 162.05 93.35) (width 0.4) (layer F.Cu) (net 9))
 (segment (start 151.2 92.5) (end 150.5 92.5) (width 0.4) (layer F.Cu) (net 4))
 (segment (start 151.74 93.04) (end 151.2 92.5) (width 0.4) (layer F.Cu) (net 4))
 (segment (start 153 93.04) (end 151.74 93.04) (width 0.4) (layer F.Cu) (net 4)))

